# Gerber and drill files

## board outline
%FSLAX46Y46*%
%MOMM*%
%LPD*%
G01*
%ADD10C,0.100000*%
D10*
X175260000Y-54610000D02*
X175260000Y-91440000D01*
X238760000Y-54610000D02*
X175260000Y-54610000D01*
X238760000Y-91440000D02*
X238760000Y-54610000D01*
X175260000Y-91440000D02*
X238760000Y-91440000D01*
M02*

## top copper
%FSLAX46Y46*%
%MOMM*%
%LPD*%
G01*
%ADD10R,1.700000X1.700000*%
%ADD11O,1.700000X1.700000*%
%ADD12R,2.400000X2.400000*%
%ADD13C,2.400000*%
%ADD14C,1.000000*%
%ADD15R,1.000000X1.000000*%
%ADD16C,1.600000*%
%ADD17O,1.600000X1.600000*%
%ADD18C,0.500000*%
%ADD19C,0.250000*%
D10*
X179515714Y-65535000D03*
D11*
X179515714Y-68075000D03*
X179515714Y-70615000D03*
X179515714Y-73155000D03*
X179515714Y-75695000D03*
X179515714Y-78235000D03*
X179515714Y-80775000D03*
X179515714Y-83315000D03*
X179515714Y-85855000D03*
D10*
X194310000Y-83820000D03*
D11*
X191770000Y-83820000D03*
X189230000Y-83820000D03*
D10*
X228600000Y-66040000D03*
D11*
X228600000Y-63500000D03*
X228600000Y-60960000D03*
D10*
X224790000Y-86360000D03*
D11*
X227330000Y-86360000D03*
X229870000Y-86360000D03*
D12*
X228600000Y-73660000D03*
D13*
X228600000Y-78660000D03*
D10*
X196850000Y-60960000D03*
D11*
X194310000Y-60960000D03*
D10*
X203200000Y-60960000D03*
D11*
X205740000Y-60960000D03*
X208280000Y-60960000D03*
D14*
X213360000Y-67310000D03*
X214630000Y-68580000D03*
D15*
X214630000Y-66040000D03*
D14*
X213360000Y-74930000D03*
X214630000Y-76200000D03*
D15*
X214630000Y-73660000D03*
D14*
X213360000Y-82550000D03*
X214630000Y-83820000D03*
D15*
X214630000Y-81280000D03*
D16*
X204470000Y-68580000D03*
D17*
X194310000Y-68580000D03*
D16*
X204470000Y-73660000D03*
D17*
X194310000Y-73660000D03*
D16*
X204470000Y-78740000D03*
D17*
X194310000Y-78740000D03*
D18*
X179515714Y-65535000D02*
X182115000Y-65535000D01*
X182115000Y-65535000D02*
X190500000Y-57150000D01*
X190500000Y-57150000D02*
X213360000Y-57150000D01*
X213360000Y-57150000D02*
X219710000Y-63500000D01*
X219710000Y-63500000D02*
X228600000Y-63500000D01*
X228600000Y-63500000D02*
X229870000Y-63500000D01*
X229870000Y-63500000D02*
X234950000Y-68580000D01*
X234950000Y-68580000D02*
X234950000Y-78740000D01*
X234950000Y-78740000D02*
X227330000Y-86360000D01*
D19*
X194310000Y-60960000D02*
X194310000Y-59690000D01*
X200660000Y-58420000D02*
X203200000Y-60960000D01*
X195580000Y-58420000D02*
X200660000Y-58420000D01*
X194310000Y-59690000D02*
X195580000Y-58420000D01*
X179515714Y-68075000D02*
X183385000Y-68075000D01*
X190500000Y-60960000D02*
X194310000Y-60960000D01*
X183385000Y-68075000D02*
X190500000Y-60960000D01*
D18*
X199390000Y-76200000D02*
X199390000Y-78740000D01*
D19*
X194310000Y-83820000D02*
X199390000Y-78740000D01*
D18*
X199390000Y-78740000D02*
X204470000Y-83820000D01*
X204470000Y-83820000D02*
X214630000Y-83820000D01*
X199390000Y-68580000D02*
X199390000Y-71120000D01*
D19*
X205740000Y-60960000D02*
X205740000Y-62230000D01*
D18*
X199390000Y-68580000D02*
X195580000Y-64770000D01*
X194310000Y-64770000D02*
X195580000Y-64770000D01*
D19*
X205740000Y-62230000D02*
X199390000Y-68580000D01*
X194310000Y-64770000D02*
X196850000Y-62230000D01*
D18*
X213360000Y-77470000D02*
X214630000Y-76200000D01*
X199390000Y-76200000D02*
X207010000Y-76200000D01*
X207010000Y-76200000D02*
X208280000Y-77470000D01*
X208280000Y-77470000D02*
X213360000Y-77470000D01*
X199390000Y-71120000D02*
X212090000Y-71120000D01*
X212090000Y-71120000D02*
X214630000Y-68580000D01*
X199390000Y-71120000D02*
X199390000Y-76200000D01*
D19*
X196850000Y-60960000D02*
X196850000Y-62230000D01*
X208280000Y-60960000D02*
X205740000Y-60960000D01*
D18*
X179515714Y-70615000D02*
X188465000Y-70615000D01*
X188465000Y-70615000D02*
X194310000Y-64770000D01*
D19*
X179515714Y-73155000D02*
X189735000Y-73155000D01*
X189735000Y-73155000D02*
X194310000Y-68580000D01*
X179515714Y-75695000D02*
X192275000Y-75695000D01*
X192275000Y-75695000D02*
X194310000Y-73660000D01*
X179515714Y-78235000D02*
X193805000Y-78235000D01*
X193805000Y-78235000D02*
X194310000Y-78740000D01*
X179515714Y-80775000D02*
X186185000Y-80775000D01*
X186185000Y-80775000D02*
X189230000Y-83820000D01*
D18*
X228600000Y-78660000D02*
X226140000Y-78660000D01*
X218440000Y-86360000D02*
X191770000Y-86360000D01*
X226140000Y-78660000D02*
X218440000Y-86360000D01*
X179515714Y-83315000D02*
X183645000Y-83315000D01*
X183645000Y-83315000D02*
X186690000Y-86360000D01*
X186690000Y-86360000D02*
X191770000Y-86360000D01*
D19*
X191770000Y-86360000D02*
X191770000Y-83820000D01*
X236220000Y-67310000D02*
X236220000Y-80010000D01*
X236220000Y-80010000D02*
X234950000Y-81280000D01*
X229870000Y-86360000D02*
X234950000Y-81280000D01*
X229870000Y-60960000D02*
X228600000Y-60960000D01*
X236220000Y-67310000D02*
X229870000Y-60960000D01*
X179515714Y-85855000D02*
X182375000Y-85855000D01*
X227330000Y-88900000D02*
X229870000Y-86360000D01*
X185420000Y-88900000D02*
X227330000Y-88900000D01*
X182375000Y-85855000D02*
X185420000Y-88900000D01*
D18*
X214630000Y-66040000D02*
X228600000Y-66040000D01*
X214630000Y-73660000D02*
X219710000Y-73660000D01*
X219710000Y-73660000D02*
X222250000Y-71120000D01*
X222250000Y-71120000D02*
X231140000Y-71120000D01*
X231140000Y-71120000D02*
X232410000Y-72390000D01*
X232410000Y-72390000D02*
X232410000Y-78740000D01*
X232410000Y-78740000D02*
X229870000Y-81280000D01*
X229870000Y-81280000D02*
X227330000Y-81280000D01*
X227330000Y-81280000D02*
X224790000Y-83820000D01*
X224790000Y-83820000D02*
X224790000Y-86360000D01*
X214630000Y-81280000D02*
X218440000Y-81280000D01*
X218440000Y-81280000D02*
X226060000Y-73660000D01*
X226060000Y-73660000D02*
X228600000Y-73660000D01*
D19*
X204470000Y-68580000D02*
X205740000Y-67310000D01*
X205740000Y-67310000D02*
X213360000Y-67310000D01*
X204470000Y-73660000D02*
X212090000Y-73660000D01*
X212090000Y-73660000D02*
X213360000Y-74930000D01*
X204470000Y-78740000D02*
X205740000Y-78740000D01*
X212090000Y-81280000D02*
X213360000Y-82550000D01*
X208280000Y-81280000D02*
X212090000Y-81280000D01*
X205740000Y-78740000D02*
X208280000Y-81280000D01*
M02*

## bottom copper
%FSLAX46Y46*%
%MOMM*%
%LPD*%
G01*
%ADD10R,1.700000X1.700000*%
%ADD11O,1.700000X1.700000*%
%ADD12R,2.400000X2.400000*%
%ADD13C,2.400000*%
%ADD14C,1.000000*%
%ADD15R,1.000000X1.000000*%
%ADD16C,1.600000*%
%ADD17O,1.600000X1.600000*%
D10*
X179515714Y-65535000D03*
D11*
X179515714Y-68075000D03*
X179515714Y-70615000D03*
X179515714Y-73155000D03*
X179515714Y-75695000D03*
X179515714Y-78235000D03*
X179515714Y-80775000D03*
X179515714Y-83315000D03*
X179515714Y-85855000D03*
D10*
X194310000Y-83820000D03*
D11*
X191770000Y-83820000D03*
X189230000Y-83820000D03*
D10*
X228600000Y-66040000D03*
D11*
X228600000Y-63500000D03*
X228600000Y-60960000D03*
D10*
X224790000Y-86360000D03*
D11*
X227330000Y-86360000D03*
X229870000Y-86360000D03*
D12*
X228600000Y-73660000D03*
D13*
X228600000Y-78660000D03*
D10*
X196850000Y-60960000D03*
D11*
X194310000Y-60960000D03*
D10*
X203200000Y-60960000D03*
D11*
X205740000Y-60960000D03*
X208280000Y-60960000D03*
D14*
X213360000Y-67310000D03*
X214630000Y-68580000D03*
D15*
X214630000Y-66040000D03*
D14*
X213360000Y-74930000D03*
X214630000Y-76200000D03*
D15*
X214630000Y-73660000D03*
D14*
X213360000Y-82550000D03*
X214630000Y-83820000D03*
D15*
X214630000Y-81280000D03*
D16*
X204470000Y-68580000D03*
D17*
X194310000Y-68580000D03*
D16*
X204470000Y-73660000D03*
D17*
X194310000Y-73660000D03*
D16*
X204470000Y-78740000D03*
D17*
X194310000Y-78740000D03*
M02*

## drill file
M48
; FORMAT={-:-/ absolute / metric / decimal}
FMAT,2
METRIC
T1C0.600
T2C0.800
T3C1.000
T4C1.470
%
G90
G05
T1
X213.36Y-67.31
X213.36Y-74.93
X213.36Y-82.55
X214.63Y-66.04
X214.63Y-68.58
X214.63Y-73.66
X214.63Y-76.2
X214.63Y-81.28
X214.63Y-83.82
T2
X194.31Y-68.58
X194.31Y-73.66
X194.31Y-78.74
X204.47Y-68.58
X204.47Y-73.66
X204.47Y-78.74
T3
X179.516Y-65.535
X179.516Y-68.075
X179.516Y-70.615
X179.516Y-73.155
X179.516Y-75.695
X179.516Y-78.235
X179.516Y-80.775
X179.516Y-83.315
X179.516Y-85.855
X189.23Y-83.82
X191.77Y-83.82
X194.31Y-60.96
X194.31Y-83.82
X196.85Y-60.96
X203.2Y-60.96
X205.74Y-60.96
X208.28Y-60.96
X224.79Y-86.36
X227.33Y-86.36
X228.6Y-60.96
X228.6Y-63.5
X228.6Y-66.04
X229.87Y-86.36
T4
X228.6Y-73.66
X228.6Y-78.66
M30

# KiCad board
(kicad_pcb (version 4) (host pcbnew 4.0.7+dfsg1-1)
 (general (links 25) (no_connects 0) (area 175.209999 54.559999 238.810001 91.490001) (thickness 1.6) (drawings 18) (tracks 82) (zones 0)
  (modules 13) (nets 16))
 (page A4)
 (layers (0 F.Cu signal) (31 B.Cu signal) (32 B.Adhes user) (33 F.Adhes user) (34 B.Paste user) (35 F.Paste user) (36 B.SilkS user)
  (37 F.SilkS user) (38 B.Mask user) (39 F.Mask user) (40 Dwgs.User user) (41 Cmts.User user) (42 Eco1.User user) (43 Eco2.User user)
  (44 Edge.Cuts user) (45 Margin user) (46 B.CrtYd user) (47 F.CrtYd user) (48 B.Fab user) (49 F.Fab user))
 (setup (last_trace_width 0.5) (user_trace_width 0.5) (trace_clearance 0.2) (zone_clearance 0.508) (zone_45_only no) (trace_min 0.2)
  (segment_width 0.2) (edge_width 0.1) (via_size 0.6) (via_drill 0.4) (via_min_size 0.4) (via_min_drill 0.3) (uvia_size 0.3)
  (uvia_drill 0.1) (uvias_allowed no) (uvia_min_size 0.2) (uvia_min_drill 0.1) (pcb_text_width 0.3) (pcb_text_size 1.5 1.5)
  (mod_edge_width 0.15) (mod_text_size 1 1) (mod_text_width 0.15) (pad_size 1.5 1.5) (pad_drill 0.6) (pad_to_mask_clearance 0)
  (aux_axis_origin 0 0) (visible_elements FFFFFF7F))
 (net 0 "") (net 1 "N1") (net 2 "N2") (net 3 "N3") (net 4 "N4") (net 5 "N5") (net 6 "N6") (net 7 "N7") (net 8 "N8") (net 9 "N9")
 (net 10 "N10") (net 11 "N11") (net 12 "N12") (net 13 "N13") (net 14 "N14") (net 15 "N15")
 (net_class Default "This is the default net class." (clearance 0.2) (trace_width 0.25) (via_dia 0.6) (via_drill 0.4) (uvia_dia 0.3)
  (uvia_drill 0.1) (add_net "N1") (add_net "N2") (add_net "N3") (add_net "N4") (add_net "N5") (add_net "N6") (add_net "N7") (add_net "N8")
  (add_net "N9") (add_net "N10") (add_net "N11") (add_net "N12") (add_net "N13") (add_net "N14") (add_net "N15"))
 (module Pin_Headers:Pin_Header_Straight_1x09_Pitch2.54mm (layer F.Cu) (at 179.515714 65.535)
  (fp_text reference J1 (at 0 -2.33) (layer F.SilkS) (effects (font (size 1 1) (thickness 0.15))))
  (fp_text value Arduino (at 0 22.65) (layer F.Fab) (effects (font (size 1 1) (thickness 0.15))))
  (pad 1 thru_hole rect (at 0 0) (size 1.7 1.7) (drill 1) (layers *.Cu *.Mask) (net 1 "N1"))
  (pad 2 thru_hole oval (at 0 2.54) (size 1.7 1.7) (drill 1) (layers *.Cu *.Mask) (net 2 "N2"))
  (pad 3 thru_hole oval (at 0 5.08) (size 1.7 1.7) (drill 1) (layers *.Cu *.Mask) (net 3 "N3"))
  (pad 4 thru_hole oval (at 0 7.62) (size 1.7 1.7) (drill 1) (layers *.Cu *.Mask) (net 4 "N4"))
  (pad 5 thru_hole oval (at 0 10.16) (size 1.7 1.7) (drill 1) (layers *.Cu *.Mask) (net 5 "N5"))
  (pad 6 thru_hole oval (at 0 12.7) (size 1.7 1.7) (drill 1) (layers *.Cu *.Mask) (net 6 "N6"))
  (pad 7 thru_hole oval (at 0 15.24) (size 1.7 1.7) (drill 1) (layers *.Cu *.Mask) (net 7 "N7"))
  (pad 8 thru_hole oval (at 0 17.78) (size 1.7 1.7) (drill 1) (layers *.Cu *.Mask) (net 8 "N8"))
  (pad 9 thru_hole oval (at 0 20.32) (size 1.7 1.7) (drill 1) (layers *.Cu *.Mask) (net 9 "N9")))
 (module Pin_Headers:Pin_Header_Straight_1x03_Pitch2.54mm (layer F.Cu) (at 194.31 83.82 270)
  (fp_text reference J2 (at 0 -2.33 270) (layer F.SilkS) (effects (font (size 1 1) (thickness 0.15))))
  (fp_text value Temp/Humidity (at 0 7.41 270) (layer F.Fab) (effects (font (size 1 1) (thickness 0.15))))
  (pad 1 thru_hole rect (at 0 0 270) (size 1.7 1.7) (drill 1) (layers *.Cu *.Mask) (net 3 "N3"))
  (pad 2 thru_hole oval (at 0 2.54 270) (size 1.7 1.7) (drill 1) (layers *.Cu *.Mask) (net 8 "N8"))
  (pad 3 thru_hole oval (at 0 5.08 270) (size 1.7 1.7) (drill 1) (layers *.Cu *.Mask) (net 7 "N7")))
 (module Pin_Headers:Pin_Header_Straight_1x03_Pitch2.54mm (layer F.Cu) (at 228.6 66.04 180)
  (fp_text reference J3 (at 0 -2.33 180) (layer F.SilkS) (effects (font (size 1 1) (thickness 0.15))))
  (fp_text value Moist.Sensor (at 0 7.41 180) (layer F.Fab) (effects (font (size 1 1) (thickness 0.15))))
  (pad 1 thru_hole rect (at 0 0 180) (size 1.7 1.7) (drill 1) (layers *.Cu *.Mask) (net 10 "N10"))
  (pad 2 thru_hole oval (at 0 2.54 180) (size 1.7 1.7) (drill 1) (layers *.Cu *.Mask) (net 1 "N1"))
  (pad 3 thru_hole oval (at 0 5.08 180) (size 1.7 1.7) (drill 1) (layers *.Cu *.Mask) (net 9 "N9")))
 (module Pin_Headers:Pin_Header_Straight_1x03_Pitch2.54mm (layer F.Cu) (at 224.79 86.36 90)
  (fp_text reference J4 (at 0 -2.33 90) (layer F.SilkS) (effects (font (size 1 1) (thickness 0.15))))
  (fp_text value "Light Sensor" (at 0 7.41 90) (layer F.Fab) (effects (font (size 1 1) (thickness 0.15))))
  (pad 1 thru_hole rect (at 0 0 90) (size 1.7 1.7) (drill 1) (layers *.Cu *.Mask) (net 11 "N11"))
  (pad 2 thru_hole oval (at 0 2.54 90) (size 1.7 1.7) (drill 1) (layers *.Cu *.Mask) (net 1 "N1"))
  (pad 3 thru_hole oval (at 0 5.08 90) (size 1.7 1.7) (drill 1) (layers *.Cu *.Mask) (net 9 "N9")))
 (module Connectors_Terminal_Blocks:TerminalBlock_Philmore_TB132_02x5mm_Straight (layer F.Cu) (at 228.6 73.66 270)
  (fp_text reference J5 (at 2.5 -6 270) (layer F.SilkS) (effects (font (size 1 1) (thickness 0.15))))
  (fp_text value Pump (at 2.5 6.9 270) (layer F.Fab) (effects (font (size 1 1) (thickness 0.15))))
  (pad 1 thru_hole rect (at 0 0 270) (size 2.4 2.4) (drill 1.47) (layers *.Cu *.Mask) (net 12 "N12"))
  (pad 2 thru_hole circle (at 5 0 270) (size 2.4 2.4) (drill 1.47) (layers *.Cu *.Mask) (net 8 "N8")))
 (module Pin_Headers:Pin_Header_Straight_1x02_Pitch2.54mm (layer F.Cu) (at 196.85 60.96 270)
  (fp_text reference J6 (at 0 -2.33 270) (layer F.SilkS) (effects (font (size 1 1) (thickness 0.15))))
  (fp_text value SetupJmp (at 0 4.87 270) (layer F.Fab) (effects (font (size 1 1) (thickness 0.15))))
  (pad 1 thru_hole rect (at 0 0 270) (size 1.7 1.7) (drill 1) (layers *.Cu *.Mask) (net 3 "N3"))
  (pad 2 thru_hole oval (at 0 2.54 270) (size 1.7 1.7) (drill 1) (layers *.Cu *.Mask) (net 2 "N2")))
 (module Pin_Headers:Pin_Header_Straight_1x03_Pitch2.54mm (layer F.Cu) (at 203.2 60.96 90)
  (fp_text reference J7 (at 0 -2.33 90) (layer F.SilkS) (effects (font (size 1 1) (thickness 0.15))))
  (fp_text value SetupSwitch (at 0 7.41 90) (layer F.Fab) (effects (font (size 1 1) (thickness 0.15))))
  (pad 1 thru_hole rect (at 0 0 90) (size 1.7 1.7) (drill 1) (layers *.Cu *.Mask) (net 2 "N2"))
  (pad 2 thru_hole oval (at 0 2.54 90) (size 1.7 1.7) (drill 1) (layers *.Cu *.Mask) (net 3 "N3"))
  (pad 3 thru_hole oval (at 0 5.08 90) (size 1.7 1.7) (drill 1) (layers *.Cu *.Mask) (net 3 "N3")))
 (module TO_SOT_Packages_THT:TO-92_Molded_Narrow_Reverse (layer F.Cu) (at 214.63 66.04 270)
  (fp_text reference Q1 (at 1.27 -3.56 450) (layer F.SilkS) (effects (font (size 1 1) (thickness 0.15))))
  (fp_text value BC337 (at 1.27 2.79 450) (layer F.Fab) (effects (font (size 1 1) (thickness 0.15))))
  (pad 2 thru_hole circle (at 1.27 1.27) (size 1 1) (drill 0.6) (layers *.Cu *.Mask) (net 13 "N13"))
  (pad 3 thru_hole circle (at 2.54 0) (size 1 1) (drill 0.6) (layers *.Cu *.Mask) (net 3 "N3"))
  (pad 1 thru_hole rect (at 0 0) (size 1 1) (drill 0.6) (layers *.Cu *.Mask) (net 10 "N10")))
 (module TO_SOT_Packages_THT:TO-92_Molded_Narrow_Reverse (layer F.Cu) (at 214.63 73.66 270)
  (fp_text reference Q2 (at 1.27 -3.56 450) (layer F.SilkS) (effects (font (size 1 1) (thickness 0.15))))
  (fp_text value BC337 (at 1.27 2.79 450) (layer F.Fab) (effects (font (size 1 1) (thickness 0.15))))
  (pad 2 thru_hole circle (at 1.27 1.27) (size 1 1) (drill 0.6) (layers *.Cu *.Mask) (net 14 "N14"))
  (pad 3 thru_hole circle (at 2.54 0) (size 1 1) (drill 0.6) (layers *.Cu *.Mask) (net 3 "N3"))
  (pad 1 thru_hole rect (at 0 0) (size 1 1) (drill 0.6) (layers *.Cu *.Mask) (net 11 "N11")))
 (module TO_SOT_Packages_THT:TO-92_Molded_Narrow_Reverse (layer F.Cu) (at 214.63 81.28 270)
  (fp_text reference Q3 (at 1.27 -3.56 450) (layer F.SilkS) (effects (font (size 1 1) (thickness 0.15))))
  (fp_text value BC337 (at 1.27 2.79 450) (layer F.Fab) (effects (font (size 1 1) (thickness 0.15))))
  (pad 2 thru_hole circle (at 1.27 1.27) (size 1 1) (drill 0.6) (layers *.Cu *.Mask) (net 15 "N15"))
  (pad 3 thru_hole circle (at 2.54 0) (size 1 1) (drill 0.6) (layers *.Cu *.Mask) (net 3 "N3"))
  (pad 1 thru_hole rect (at 0 0) (size 1 1) (drill 0.6) (layers *.Cu *.Mask) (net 12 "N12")))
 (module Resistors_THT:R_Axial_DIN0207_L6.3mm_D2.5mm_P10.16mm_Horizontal (layer F.Cu) (at 204.47 68.58 180)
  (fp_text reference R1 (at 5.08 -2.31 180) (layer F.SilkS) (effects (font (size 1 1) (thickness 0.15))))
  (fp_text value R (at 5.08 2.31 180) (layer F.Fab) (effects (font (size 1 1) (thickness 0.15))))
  (pad 1 thru_hole circle (at 0 0 180) (size 1.6 1.6) (drill 0.8) (layers *.Cu *.Mask) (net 13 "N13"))
  (pad 2 thru_hole oval (at 10.16 0 180) (size 1.6 1.6) (drill 0.8) (layers *.Cu *.Mask) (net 4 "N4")))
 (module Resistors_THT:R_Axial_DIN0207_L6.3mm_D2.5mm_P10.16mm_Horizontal (layer F.Cu) (at 204.47 73.66 180)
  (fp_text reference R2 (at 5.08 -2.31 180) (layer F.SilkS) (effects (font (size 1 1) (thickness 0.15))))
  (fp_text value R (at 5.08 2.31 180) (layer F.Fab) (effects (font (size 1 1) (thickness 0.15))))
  (pad 1 thru_hole circle (at 0 0 180) (size 1.6 1.6) (drill 0.8) (layers *.Cu *.Mask) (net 14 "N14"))
  (pad 2 thru_hole oval (at 10.16 0 180) (size 1.6 1.6) (drill 0.8) (layers *.Cu *.Mask) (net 5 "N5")))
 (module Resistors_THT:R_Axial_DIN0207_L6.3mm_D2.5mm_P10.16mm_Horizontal (layer F.Cu) (at 204.47 78.74 180)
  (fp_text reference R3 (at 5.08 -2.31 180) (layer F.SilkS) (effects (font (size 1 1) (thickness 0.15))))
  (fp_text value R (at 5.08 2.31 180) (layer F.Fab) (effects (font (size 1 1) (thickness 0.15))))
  (pad 1 thru_hole circle (at 0 0 180) (size 1.6 1.6) (drill 0.8) (layers *.Cu *.Mask) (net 15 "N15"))
  (pad 2 thru_hole oval (at 10.16 0 180) (size 1.6 1.6) (drill 0.8) (layers *.Cu *.Mask) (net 6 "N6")))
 (gr_line (start 175.26 54.61) (end 175.26 91.44) (angle 90) (layer Edge.Cuts) (width 0.1))
 (gr_line (start 238.76 54.61) (end 175.26 54.61) (angle 90) (layer Edge.Cuts) (width 0.1))
 (gr_line (start 238.76 91.44) (end 238.76 54.61) (angle 90) (layer Edge.Cuts) (width 0.1))
 (gr_line (start 175.26 91.44) (end 238.76 91.44) (angle 90) (layer Edge.Cuts) (width 0.1))
 (segment (start 179.515714 65.535) (end 182.115 65.535) (width 0.5) (layer F.Cu) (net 1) (status 400000))
 (segment (start 182.115 65.535) (end 190.5 57.15) (width 0.5) (layer F.Cu) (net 1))
 (segment (start 190.5 57.15) (end 213.36 57.15) (width 0.5) (layer F.Cu) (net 1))
 (segment (start 213.36 57.15) (end 219.71 63.5) (width 0.5) (layer F.Cu) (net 1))
 (segment (start 219.71 63.5) (end 228.6 63.5) (width 0.5) (layer F.Cu) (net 1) (status 800000))
 (segment (start 228.6 63.5) (end 229.87 63.5) (width 0.5) (layer F.Cu) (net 1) (status 400000))
 (segment (start 229.87 63.5) (end 234.95 68.58) (width 0.5) (layer F.Cu) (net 1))
 (segment (start 234.95 68.58) (end 234.95 78.74) (width 0.5) (layer F.Cu) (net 1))
 (segment (start 234.95 78.74) (end 227.33 86.36) (width 0.5) (layer F.Cu) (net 1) (status 800000))
 (segment (start 194.31 60.96) (end 194.31 59.69) (width 0.25) (layer F.Cu) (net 2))
 (segment (start 200.66 58.42) (end 203.2 60.96) (width 0.25) (layer F.Cu) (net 2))
 (segment (start 195.58 58.42) (end 200.66 58.42) (width 0.25) (layer F.Cu) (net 2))
 (segment (start 194.31 59.69) (end 195.58 58.42) (width 0.25) (layer F.Cu) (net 2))
 (segment (start 179.515714 68.075) (end 183.385 68.075) (width 0.25) (layer F.Cu) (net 2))
 (segment (start 190.5 60.96) (end 194.31 60.96) (width 0.25) (layer F.Cu) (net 2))
 (segment (start 183.385 68.075) (end 190.5 60.96) (width 0.25) (layer F.Cu) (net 2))
 (segment (start 199.39 76.2) (end 199.39 78.74) (width 0.5) (layer F.Cu) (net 3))
 (segment (start 194.31 83.82) (end 199.39 78.74) (width 0.25) (layer F.Cu) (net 3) (status 400000))
 (segment (start 199.39 78.74) (end 204.47 83.82) (width 0.5) (layer F.Cu) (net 3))
 (segment (start 204.47 83.82) (end 214.63 83.82) (width 0.5) (layer F.Cu) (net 3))
 (segment (start 199.39 68.58) (end 199.39 71.12) (width 0.5) (layer F.Cu) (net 3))
 (segment (start 205.74 60.96) (end 205.74 62.23) (width 0.25) (layer F.Cu) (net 3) (status 400000))
 (segment (start 199.39 68.58) (end 195.58 64.77) (width 0.5) (layer F.Cu) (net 3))
 (segment (start 194.31 64.77) (end 195.58 64.77) (width 0.5) (layer F.Cu) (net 3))
 (segment (start 205.74 62.23) (end 199.39 68.58) (width 0.25) (layer F.Cu) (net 3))
 (segment (start 194.31 64.77) (end 196.85 62.23) (width 0.25) (layer F.Cu) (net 3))
 (segment (start 213.36 77.47) (end 214.63 76.2) (width 0.5) (layer F.Cu) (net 3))
 (segment (start 199.39 76.2) (end 207.01 76.2) (width 0.5) (layer F.Cu) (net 3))
 (segment (start 207.01 76.2) (end 208.28 77.47) (width 0.5) (layer F.Cu) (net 3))
 (segment (start 208.28 77.47) (end 213.36 77.47) (width 0.5) (layer F.Cu) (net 3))
 (segment (start 199.39 71.12) (end 212.09 71.12) (width 0.5) (layer F.Cu) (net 3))
 (segment (start 212.09 71.12) (end 214.63 68.58) (width 0.5) (layer F.Cu) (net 3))
 (segment (start 199.39 71.12) (end 199.39 76.2) (width 0.5) (layer F.Cu) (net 3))
 (segment (start 196.85 60.96) (end 196.85 62.23) (width 0.25) (layer F.Cu) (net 3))
 (segment (start 208.28 60.96) (end 205.74 60.96) (width 0.25) (layer F.Cu) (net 3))
 (segment (start 179.515714 70.615) (end 188.465 70.615) (width 0.5) (layer F.Cu) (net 3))
 (segment (start 188.465 70.615) (end 194.31 64.77) (width 0.5) (layer F.Cu) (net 3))
 (segment (start 179.515714 73.155) (end 189.735 73.155) (width 0.25) (layer F.Cu) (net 4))
 (segment (start 189.735 73.155) (end 194.31 68.58) (width 0.25) (layer F.Cu) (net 4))
 (segment (start 179.515714 75.695) (end 192.275 75.695) (width 0.25) (layer F.Cu) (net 5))
 (segment (start 192.275 75.695) (end 194.31 73.66) (width 0.25) (layer F.Cu) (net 5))
 (segment (start 179.515714 78.235) (end 193.805 78.235) (width 0.25) (layer F.Cu) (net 6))
 (segment (start 193.805 78.235) (end 194.31 78.74) (width 0.25) (layer F.Cu) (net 6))
 (segment (start 179.515714 80.775) (end 186.185 80.775) (width 0.25) (layer F.Cu) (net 7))
 (segment (start 186.185 80.775) (end 189.23 83.82) (width 0.25) (layer F.Cu) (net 7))
 (segment (start 228.6 78.66) (end 226.14 78.66) (width 0.5) (layer F.Cu) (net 8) (status 400000))
 (segment (start 218.44 86.36) (end 191.77 86.36) (width 0.5) (layer F.Cu) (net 8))
 (segment (start 226.14 78.66) (end 218.44 86.36) (width 0.5) (layer F.Cu) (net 8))
 (segment (start 179.515714 83.315) (end 183.645 83.315) (width 0.5) (layer F.Cu) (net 8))
 (segment (start 183.645 83.315) (end 186.69 86.36) (width 0.5) (layer F.Cu) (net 8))
 (segment (start 186.69 86.36) (end 191.77 86.36) (width 0.5) (layer F.Cu) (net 8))
 (segment (start 191.77 86.36) (end 191.77 83.82) (width 0.25) (layer F.Cu) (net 8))
 (segment (start 236.22 67.31) (end 236.22 80.01) (width 0.25) (layer F.Cu) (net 9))
 (segment (start 236.22 80.01) (end 234.95 81.28) (width 0.25) (layer F.Cu) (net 9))
 (segment (start 229.87 86.36) (end 234.95 81.28) (width 0.25) (layer F.Cu) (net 9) (status 400000))
 (segment (start 229.87 60.96) (end 228.6 60.96) (width 0.25) (layer F.Cu) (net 9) (status 800000))
 (segment (start 236.22 67.31) (end 229.87 60.96) (width 0.25) (layer F.Cu) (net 9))
 (segment (start 179.515714 85.855) (end 182.375 85.855) (width 0.25) (layer F.Cu) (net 9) (status 400000))
 (segment (start 227.33 88.9) (end 229.87 86.36) (width 0.25) (layer F.Cu) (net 9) (status 800000))
 (segment (start 185.42 88.9) (end 227.33 88.9) (width 0.25) (layer F.Cu) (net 9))
 (segment (start 182.375 85.855) (end 185.42 88.9) (width 0.25) (layer F.Cu) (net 9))
 (segment (start 214.63 66.04) (end 228.6 66.04) (width 0.5) (layer F.Cu) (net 10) (status C00000))
 (segment (start 214.63 73.66) (end 219.71 73.66) (width 0.5) (layer F.Cu) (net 11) (status 400000))
 (segment (start 219.71 73.66) (end 222.25 71.12) (width 0.5) (layer F.Cu) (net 11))
 (segment (start 222.25 71.12) (end 231.14 71.12) (width 0.5) (layer F.Cu) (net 11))
 (segment (start 231.14 71.12) (end 232.41 72.39) (width 0.5) (layer F.Cu) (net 11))
 (segment (start 232.41 72.39) (end 232.41 78.74) (width 0.5) (layer F.Cu) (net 11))
 (segment (start 232.41 78.74) (end 229.87 81.28) (width 0.5) (layer F.Cu) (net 11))
 (segment (start 229.87 81.28) (end 227.33 81.28) (width 0.5) (layer F.Cu) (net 11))
 (segment (start 227.33 81.28) (end 224.79 83.82) (width 0.5) (layer F.Cu) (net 11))
 (segment (start 224.79 83.82) (end 224.79 86.36) (width 0.5) (layer F.Cu) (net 11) (status 800000))
 (segment (start 214.63 81.28) (end 218.44 81.28) (width 0.5) (layer F.Cu) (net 12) (status 400000))
 (segment (start 218.44 81.28) (end 226.06 73.66) (width 0.5) (layer F.Cu) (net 12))
 (segment (start 226.06 73.66) (end 228.6 73.66) (width 0.5) (layer F.Cu) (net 12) (status 800000))
 (segment (start 204.47 68.58) (end 205.74 67.31) (width 0.25) (layer F.Cu) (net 13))
 (segment (start 205.74 67.31) (end 213.36 67.31) (width 0.25) (layer F.Cu) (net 13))
 (segment (start 204.47 73.66) (end 212.09 73.66) (width 0.25) (layer F.Cu) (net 14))
 (segment (start 212.09 73.66) (end 213.36 74.93) (width 0.25) (layer F.Cu) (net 14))
 (segment (start 204.47 78.74) (end 205.74 78.74) (width 0.25) (layer F.Cu) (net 15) (status 400000))
 (segment (start 212.09 81.28) (end 213.36 82.55) (width 0.25) (layer F.Cu) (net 15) (status 800000))
 (segment (start 208.28 81.28) (end 212.09 81.28) (width 0.25) (layer F.Cu) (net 15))
 (segment (start 205.74 78.74) (end 208.28 81.28) (width 0.25) (layer F.Cu) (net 15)))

